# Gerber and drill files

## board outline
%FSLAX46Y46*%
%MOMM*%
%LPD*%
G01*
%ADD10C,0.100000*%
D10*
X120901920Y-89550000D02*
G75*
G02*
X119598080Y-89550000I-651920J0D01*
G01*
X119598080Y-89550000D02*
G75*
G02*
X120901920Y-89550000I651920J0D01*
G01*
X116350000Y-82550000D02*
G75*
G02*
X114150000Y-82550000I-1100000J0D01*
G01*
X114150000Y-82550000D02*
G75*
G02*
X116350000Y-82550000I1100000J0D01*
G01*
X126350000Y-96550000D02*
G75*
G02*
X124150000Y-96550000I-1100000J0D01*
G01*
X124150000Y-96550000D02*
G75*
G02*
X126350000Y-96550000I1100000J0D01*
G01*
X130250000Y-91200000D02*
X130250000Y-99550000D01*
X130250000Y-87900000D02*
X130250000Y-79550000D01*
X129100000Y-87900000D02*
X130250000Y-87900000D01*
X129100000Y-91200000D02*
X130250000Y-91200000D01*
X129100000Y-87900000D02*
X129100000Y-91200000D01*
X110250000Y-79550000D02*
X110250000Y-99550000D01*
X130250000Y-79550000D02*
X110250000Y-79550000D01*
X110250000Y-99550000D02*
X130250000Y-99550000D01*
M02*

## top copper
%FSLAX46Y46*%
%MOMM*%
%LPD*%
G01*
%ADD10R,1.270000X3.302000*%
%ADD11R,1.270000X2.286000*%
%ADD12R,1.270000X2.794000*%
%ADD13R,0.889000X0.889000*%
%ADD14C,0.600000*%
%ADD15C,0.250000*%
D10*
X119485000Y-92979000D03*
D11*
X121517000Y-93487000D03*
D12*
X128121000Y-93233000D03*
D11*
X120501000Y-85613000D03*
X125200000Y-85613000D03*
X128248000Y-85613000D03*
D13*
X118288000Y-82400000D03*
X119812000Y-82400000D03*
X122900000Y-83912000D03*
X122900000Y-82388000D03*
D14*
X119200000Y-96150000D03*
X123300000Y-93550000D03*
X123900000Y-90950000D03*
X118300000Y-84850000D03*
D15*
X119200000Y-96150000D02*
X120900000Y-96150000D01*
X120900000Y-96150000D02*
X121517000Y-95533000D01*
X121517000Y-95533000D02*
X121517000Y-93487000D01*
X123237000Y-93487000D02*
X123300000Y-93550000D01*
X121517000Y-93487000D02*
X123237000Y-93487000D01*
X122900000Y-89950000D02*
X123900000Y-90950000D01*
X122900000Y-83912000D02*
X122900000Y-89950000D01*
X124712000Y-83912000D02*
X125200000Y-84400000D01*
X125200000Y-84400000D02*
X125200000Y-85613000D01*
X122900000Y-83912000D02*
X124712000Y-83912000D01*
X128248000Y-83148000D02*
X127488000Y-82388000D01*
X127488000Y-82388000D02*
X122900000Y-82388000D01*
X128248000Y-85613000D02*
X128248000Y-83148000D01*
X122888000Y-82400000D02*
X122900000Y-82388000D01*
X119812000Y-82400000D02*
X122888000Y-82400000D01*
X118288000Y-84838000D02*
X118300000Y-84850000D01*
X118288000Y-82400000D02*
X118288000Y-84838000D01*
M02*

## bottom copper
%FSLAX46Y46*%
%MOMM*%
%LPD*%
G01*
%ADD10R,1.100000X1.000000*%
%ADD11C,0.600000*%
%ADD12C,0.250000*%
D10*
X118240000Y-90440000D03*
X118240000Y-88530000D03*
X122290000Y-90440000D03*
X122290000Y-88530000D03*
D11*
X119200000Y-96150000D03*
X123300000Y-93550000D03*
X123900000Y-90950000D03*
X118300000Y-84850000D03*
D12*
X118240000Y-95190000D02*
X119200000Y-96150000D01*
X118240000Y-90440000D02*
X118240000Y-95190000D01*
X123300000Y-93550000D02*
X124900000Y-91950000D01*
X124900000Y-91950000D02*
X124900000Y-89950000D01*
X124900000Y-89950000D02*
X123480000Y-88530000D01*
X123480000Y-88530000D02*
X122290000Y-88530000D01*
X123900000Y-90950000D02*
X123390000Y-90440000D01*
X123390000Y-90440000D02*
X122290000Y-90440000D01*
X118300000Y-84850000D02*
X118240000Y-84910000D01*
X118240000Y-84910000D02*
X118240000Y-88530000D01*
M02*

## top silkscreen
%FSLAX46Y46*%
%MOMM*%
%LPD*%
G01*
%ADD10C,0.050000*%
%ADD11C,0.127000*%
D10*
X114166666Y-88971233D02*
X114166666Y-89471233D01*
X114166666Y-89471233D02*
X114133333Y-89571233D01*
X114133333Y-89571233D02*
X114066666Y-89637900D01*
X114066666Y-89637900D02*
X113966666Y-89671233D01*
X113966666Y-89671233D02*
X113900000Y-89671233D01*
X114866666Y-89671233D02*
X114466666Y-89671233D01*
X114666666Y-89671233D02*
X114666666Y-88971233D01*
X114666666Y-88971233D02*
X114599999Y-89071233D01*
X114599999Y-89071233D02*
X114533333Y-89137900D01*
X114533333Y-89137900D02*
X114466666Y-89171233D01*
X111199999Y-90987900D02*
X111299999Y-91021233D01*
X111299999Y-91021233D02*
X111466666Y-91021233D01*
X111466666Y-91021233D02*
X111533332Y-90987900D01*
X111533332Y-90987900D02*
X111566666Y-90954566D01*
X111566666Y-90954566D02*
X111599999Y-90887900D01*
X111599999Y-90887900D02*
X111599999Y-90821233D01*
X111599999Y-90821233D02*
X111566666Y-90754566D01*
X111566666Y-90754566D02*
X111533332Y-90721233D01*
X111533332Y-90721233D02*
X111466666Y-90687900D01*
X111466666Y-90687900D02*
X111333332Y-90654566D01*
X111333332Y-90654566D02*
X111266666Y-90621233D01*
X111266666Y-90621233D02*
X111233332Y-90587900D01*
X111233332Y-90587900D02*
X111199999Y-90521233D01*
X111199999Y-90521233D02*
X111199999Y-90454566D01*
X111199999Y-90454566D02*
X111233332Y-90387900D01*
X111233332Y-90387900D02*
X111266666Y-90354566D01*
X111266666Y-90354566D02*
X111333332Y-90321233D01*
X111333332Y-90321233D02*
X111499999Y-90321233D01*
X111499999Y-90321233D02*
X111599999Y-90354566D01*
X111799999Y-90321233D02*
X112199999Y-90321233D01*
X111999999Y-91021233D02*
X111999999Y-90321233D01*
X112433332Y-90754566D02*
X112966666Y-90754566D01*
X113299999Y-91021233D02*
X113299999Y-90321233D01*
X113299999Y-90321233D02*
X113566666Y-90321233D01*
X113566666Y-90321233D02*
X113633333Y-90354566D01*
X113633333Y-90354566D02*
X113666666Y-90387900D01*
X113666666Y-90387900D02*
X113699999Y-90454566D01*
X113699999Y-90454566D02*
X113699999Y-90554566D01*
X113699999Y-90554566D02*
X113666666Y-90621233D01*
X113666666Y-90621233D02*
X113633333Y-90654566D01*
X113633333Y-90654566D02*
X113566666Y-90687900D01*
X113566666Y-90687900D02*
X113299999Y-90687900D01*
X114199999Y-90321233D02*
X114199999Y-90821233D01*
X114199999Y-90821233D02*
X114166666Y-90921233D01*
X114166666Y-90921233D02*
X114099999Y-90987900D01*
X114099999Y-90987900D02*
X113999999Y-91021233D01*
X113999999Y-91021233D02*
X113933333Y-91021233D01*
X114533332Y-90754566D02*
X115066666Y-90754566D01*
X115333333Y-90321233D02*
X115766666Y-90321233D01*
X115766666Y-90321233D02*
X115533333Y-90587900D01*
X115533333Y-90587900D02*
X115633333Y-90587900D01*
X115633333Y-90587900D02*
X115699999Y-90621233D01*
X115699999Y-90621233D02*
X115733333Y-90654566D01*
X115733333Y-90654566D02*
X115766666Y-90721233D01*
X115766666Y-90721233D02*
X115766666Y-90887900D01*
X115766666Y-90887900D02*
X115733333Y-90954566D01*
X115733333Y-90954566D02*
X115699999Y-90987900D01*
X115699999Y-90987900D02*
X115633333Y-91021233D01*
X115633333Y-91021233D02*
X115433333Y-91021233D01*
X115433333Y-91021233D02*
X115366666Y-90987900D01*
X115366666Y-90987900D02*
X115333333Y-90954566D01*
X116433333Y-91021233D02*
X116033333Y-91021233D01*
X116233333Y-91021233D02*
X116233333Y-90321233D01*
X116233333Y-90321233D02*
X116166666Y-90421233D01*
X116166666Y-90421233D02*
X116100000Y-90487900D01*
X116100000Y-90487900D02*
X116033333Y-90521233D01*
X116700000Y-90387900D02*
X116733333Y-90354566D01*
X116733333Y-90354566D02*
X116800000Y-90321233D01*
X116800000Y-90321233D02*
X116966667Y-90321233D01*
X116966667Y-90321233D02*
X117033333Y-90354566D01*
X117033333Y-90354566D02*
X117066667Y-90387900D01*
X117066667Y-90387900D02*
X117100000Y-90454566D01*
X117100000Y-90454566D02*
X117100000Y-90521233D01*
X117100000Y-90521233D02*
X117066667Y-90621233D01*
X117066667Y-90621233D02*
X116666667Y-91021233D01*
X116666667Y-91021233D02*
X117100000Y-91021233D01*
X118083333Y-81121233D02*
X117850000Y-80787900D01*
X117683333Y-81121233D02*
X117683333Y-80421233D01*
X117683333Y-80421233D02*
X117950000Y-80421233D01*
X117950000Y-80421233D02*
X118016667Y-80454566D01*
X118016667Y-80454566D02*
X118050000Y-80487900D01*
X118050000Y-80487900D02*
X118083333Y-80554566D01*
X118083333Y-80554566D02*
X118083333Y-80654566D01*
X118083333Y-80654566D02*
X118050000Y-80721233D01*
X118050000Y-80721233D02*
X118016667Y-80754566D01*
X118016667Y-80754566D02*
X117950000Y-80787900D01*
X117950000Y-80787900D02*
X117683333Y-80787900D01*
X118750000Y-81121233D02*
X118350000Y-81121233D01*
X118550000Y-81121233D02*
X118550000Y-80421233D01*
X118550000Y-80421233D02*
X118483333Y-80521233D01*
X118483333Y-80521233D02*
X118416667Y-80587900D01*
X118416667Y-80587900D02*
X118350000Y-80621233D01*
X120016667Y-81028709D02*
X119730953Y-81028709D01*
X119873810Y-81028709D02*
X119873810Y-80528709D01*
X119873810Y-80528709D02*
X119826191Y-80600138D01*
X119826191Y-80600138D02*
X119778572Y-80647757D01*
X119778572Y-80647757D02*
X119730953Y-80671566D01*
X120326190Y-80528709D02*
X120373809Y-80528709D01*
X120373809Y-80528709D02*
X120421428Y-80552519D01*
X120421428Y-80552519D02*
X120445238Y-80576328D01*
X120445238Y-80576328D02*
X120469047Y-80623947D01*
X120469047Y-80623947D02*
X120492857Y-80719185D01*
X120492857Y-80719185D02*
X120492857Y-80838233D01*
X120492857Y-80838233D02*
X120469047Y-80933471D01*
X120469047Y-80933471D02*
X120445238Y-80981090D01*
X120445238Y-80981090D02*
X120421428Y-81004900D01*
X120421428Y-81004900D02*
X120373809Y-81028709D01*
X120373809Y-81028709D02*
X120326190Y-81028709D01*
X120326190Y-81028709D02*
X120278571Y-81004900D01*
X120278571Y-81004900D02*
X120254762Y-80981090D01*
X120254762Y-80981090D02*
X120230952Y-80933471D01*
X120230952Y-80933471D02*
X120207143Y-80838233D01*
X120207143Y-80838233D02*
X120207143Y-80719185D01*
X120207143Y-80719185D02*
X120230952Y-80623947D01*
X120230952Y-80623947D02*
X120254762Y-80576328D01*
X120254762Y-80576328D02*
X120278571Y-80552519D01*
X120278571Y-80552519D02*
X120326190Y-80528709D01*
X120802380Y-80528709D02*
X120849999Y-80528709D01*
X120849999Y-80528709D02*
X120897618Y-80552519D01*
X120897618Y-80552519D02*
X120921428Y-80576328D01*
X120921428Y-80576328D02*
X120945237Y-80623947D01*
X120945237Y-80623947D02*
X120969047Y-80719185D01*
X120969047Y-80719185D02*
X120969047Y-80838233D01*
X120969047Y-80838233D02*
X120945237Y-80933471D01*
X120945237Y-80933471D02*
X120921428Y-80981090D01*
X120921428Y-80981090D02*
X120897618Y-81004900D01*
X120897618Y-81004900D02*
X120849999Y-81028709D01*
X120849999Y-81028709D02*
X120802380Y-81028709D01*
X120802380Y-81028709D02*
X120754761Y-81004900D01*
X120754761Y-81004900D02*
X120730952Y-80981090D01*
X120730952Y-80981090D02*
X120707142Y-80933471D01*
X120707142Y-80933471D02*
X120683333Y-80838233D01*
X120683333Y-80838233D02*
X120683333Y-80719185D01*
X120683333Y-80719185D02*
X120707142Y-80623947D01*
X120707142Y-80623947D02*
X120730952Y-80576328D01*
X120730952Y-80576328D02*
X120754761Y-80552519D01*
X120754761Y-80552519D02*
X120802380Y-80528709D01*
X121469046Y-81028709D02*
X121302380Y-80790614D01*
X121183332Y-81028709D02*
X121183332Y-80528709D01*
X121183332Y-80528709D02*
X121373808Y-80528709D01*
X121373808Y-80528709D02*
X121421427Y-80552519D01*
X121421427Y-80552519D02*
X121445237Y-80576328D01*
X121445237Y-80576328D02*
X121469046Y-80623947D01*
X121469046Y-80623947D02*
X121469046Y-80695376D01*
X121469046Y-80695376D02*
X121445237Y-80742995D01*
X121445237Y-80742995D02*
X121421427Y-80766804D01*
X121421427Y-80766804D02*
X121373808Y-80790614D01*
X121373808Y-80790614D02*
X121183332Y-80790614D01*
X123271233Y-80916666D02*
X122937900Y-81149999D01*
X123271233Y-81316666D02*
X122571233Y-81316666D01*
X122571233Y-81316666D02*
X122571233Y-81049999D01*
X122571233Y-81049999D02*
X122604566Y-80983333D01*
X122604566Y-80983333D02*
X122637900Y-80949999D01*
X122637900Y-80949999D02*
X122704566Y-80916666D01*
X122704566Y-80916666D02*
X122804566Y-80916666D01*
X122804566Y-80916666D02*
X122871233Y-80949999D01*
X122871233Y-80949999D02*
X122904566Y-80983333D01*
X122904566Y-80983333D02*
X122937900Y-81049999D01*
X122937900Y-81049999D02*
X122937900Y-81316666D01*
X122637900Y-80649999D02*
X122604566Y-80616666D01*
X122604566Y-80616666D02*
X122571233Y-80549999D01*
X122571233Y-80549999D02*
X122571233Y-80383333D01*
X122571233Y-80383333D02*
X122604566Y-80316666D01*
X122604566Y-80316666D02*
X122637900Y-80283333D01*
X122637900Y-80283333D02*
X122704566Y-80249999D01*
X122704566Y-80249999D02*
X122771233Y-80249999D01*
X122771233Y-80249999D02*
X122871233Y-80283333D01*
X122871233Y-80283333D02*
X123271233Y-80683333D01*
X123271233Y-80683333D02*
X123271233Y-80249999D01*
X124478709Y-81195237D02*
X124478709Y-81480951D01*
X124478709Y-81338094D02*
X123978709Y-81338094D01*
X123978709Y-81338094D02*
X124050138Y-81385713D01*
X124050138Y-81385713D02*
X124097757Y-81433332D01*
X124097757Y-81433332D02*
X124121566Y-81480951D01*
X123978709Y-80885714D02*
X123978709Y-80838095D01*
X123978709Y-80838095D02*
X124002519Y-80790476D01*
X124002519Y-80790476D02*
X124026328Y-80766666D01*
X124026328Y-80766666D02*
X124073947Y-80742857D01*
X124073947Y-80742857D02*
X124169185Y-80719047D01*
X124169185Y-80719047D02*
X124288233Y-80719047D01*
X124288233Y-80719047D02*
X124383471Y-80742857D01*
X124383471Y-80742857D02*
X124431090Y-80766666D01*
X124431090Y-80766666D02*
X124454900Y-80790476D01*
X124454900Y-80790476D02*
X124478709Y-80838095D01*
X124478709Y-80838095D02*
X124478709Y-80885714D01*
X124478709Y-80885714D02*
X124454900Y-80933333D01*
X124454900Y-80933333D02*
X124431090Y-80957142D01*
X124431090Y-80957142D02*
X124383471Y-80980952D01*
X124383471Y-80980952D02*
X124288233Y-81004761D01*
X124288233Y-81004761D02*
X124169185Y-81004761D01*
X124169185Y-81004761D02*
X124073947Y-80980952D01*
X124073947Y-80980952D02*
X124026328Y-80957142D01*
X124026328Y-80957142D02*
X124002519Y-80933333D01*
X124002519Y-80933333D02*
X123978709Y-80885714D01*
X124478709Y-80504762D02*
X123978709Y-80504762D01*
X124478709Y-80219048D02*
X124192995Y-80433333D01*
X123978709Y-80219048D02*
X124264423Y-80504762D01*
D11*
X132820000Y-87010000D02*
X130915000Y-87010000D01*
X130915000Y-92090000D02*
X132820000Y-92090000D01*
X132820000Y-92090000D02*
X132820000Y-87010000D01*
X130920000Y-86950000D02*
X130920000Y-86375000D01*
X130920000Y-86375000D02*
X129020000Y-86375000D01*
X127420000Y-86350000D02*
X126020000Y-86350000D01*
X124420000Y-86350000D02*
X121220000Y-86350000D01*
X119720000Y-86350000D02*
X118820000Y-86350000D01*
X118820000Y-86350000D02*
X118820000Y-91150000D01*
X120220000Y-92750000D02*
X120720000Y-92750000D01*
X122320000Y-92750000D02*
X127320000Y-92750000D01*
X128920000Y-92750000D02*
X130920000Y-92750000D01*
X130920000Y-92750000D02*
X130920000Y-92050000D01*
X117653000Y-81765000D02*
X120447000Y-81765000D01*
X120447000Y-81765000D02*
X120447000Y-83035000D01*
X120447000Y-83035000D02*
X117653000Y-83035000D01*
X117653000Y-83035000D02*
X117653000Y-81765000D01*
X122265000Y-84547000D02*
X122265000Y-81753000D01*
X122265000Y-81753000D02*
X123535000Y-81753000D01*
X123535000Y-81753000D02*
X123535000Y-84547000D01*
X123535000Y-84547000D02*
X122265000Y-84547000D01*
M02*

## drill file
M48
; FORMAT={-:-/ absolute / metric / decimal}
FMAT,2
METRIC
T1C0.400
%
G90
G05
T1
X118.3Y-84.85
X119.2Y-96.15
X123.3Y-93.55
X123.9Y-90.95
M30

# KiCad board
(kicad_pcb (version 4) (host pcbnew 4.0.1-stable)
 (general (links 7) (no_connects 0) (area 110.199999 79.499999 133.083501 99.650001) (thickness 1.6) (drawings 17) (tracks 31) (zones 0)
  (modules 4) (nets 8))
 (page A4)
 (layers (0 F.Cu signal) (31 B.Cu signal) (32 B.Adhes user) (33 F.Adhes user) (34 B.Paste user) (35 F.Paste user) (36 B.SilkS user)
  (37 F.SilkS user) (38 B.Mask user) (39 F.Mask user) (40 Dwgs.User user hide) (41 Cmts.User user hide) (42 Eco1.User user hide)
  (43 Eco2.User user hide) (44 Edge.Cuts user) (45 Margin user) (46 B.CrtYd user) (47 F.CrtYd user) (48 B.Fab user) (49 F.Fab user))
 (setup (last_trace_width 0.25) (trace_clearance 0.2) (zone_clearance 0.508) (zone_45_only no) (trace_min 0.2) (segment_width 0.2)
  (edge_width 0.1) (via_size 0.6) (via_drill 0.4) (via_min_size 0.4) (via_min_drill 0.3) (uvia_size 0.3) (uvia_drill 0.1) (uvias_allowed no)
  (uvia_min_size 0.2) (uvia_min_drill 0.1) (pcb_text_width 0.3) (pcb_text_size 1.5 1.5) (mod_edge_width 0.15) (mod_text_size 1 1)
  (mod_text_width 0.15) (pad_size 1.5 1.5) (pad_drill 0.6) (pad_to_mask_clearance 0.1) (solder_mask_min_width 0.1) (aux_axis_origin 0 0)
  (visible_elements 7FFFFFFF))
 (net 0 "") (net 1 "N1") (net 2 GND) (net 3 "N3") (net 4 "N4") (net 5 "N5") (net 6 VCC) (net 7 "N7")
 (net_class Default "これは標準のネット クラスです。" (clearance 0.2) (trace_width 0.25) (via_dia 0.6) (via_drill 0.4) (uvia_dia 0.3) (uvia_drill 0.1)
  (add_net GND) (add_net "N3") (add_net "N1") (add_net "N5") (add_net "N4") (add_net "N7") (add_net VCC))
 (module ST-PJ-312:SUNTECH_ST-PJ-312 (layer F.Cu) (at 125.2 89.55) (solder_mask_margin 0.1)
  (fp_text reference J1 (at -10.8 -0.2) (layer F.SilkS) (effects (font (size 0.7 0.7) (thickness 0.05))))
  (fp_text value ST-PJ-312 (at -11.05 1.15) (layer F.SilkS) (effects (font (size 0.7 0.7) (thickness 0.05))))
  (fp_line (start 7.62 -2.54) (end 5.715 -2.54) (layer F.SilkS) (width 0.127))
  (fp_line (start 5.715 2.54) (end 7.62 2.54) (layer F.SilkS) (width 0.127))
  (fp_line (start 7.62 2.54) (end 7.62 -2.54) (layer F.SilkS) (width 0.127))
  (fp_line (start 5.72 -2.6) (end 5.72 -3.175) (layer F.SilkS) (width 0.127))
  (fp_line (start 5.72 -3.175) (end 3.82 -3.175) (layer F.SilkS) (width 0.127))
  (fp_line (start 2.22 -3.2) (end 0.82 -3.2) (layer F.SilkS) (width 0.127))
  (fp_line (start -0.78 -3.2) (end -3.98 -3.2) (layer F.SilkS) (width 0.127))
  (fp_line (start -5.48 -3.2) (end -6.38 -3.2) (layer F.SilkS) (width 0.127))
  (fp_line (start -6.38 -3.2) (end -6.38 1.6) (layer F.SilkS) (width 0.127))
  (fp_line (start -4.98 3.2) (end -4.48 3.2) (layer F.SilkS) (width 0.127))
  (fp_line (start -2.88 3.2) (end 2.12 3.2) (layer F.SilkS) (width 0.127))
  (fp_line (start 3.72 3.2) (end 5.72 3.2) (layer F.SilkS) (width 0.127))
  (fp_line (start 5.72 3.2) (end 5.72 2.5) (layer F.SilkS) (width 0.127))
  (pad LS smd rect (at -5.715 3.429 90) (size 3.302 1.27) (layers F.Cu F.Paste F.Mask) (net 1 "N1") (solder_mask_margin 0.2))
  (pad L smd rect (at -3.683 3.937 90) (size 2.286 1.27) (layers F.Cu F.Paste F.Mask) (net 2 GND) (solder_mask_margin 0.2))
  (pad COM2 smd rect (at 2.921 3.683 90) (size 2.794 1.27) (layers F.Cu F.Paste F.Mask) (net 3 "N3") (solder_mask_margin 0.2))
  (pad RS smd rect (at -4.699 -3.937 90) (size 2.286 1.27) (layers F.Cu F.Paste F.Mask) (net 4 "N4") (solder_mask_margin 0.2))
  (pad R smd rect (at 0 -3.937 90) (size 2.286 1.27) (layers F.Cu F.Paste F.Mask) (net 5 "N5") (solder_mask_margin 0.2))
  (pad COM1 smd rect (at 3.048 -3.937 90) (size 2.286 1.27) (layers F.Cu F.Paste F.Mask) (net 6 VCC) (solder_mask_margin 0.2)))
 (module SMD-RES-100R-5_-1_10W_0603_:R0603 (layer F.Cu) (at 119.05 82.4 90) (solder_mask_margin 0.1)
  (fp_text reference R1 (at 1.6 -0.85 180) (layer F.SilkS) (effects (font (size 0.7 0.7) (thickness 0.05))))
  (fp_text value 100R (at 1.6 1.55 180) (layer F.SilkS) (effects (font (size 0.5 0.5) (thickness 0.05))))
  (fp_line (start 0.635 -1.397) (end 0.635 1.397) (layer F.SilkS) (width 0.127))
  (fp_line (start 0.635 1.397) (end -0.635 1.397) (layer F.SilkS) (width 0.127))
  (fp_line (start -0.635 1.397) (end -0.635 -1.397) (layer F.SilkS) (width 0.127))
  (fp_line (start -0.635 -1.397) (end 0.635 -1.397) (layer F.SilkS) (width 0.127))
  (pad 1 smd rect (at 0 -0.762) (size 0.889 0.889) (layers F.Cu F.Paste F.Mask) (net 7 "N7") (solder_mask_margin 0.2))
  (pad 2 smd rect (at 0 0.762) (size 0.889 0.889) (layers F.Cu F.Paste F.Mask) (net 6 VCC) (solder_mask_margin 0.2)))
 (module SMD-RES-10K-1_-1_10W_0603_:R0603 (layer F.Cu) (at 122.9 83.15 180) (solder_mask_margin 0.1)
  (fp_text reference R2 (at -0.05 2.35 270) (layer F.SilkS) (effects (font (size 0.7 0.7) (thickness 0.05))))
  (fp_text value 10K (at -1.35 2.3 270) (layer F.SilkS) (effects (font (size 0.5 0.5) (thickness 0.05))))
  (fp_line (start 0.635 -1.397) (end 0.635 1.397) (layer F.SilkS) (width 0.127))
  (fp_line (start 0.635 1.397) (end -0.635 1.397) (layer F.SilkS) (width 0.127))
  (fp_line (start -0.635 1.397) (end -0.635 -1.397) (layer F.SilkS) (width 0.127))
  (fp_line (start -0.635 -1.397) (end 0.635 -1.397) (layer F.SilkS) (width 0.127))
  (pad 1 smd rect (at 0 -0.762 90) (size 0.889 0.889) (layers F.Cu F.Paste F.Mask) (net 5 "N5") (solder_mask_margin 0.2))
  (pad 2 smd rect (at 0 0.762 90) (size 0.889 0.889) (layers F.Cu F.Paste F.Mask) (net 6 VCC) (solder_mask_margin 0.2)))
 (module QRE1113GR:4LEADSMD (layer B.Cu) (at 120.25 89.5) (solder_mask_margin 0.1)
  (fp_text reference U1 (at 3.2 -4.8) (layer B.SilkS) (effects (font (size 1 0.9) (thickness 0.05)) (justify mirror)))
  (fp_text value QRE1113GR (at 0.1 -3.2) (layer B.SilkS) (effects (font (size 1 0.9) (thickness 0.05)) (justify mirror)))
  (pad E smd rect (at -2.01 0.94 90) (size 1 1.1) (layers B.Cu B.Paste B.Mask) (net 2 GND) (solder_mask_margin 0.2))
  (pad A smd rect (at -2.01 -0.97 90) (size 1 1.1) (layers B.Cu B.Paste B.Mask) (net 7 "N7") (solder_mask_margin 0.2))
  (pad C smd rect (at 2.04 0.94 90) (size 1 1.1) (layers B.Cu B.Paste B.Mask) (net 5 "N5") (solder_mask_margin 0.2))
  (pad K smd rect (at 2.04 -0.97 90) (size 1 1.1) (layers B.Cu B.Paste B.Mask) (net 2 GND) (solder_mask_margin 0.2)))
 (gr_circle (center 120.25 89.55) (end 120.3 88.9) (layer Edge.Cuts) (width 0.1))
 (gr_circle (center 115.25 82.55) (end 116.35 82.55) (layer Edge.Cuts) (width 0.1))
 (gr_circle (center 125.25 96.55) (end 126.35 96.55) (layer Edge.Cuts) (width 0.1))
 (gr_line (start 130.25 91.2) (end 130.25 99.55) (angle 90) (layer Edge.Cuts) (width 0.1))
 (gr_line (start 130.25 87.9) (end 130.25 79.55) (angle 90) (layer Edge.Cuts) (width 0.1))
 (gr_line (start 129.1 87.9) (end 130.25 87.9) (angle 90) (layer Edge.Cuts) (width 0.1))
 (gr_line (start 129.1 91.2) (end 130.25 91.2) (angle 90) (layer Edge.Cuts) (width 0.1))
 (gr_line (start 129.1 87.9) (end 129.1 91.2) (angle 90) (layer Edge.Cuts) (width 0.1))
 (gr_line (start 110.25 79.55) (end 110.25 99.55) (angle 90) (layer Edge.Cuts) (width 0.1))
 (gr_line (start 130.25 79.55) (end 110.25 79.55) (angle 90) (layer Edge.Cuts) (width 0.1))
 (gr_line (start 110.25 99.55) (end 130.25 99.55) (angle 90) (layer Edge.Cuts) (width 0.1))
 (segment (start 118.24 95.19) (end 119.2 96.15) (width 0.25) (layer B.Cu) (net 2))
 (via (at 119.2 96.15) (size 0.6) (layers F.Cu B.Cu) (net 2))
 (segment (start 119.2 96.15) (end 120.9 96.15) (width 0.25) (layer F.Cu) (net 2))
 (segment (start 120.9 96.15) (end 121.517 95.533) (width 0.25) (layer F.Cu) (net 2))
 (segment (start 121.517 95.533) (end 121.517 93.487) (width 0.25) (layer F.Cu) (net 2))
 (segment (start 118.24 90.44) (end 118.24 95.19) (width 0.25) (layer B.Cu) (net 2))
 (segment (start 123.237 93.487) (end 123.3 93.55) (width 0.25) (layer F.Cu) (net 2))
 (via (at 123.3 93.55) (size 0.6) (layers F.Cu B.Cu) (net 2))
 (segment (start 123.3 93.55) (end 124.9 91.95) (width 0.25) (layer B.Cu) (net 2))
 (segment (start 124.9 91.95) (end 124.9 89.95) (width 0.25) (layer B.Cu) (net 2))
 (segment (start 124.9 89.95) (end 123.48 88.53) (width 0.25) (layer B.Cu) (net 2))
 (segment (start 123.48 88.53) (end 122.29 88.53) (width 0.25) (layer B.Cu) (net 2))
 (segment (start 121.517 93.487) (end 123.237 93.487) (width 0.25) (layer F.Cu) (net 2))
 (segment (start 122.9 89.95) (end 123.9 90.95) (width 0.25) (layer F.Cu) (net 5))
 (via (at 123.9 90.95) (size 0.6) (layers F.Cu B.Cu) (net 5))
 (segment (start 123.9 90.95) (end 123.39 90.44) (width 0.25) (layer B.Cu) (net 5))
 (segment (start 123.39 90.44) (end 122.29 90.44) (width 0.25) (layer B.Cu) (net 5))
 (segment (start 122.9 83.912) (end 122.9 89.95) (width 0.25) (layer F.Cu) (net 5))
 (segment (start 124.712 83.912) (end 125.2 84.4) (width 0.25) (layer F.Cu) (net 5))
 (segment (start 125.2 84.4) (end 125.2 85.613) (width 0.25) (layer F.Cu) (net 5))
 (segment (start 122.9 83.912) (end 124.712 83.912) (width 0.25) (layer F.Cu) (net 5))
 (segment (start 128.248 83.148) (end 127.488 82.388) (width 0.25) (layer F.Cu) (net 6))
 (segment (start 127.488 82.388) (end 122.9 82.388) (width 0.25) (layer F.Cu) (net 6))
 (segment (start 128.248 85.613) (end 128.248 83.148) (width 0.25) (layer F.Cu) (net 6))
 (segment (start 122.888 82.4) (end 122.9 82.388) (width 0.25) (layer F.Cu) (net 6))
 (segment (start 119.812 82.4) (end 122.888 82.4) (width 0.25) (layer F.Cu) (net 6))
 (segment (start 118.288 84.838) (end 118.3 84.85) (width 0.25) (layer F.Cu) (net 7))
 (via (at 118.3 84.85) (size 0.6) (layers F.Cu B.Cu) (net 7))
 (segment (start 118.3 84.85) (end 118.24 84.91) (width 0.25) (layer B.Cu) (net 7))
 (segment (start 118.24 84.91) (end 118.24 88.53) (width 0.25) (layer B.Cu) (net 7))
 (segment (start 118.288 82.4) (end 118.288 84.838) (width 0.25) (layer F.Cu) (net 7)))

